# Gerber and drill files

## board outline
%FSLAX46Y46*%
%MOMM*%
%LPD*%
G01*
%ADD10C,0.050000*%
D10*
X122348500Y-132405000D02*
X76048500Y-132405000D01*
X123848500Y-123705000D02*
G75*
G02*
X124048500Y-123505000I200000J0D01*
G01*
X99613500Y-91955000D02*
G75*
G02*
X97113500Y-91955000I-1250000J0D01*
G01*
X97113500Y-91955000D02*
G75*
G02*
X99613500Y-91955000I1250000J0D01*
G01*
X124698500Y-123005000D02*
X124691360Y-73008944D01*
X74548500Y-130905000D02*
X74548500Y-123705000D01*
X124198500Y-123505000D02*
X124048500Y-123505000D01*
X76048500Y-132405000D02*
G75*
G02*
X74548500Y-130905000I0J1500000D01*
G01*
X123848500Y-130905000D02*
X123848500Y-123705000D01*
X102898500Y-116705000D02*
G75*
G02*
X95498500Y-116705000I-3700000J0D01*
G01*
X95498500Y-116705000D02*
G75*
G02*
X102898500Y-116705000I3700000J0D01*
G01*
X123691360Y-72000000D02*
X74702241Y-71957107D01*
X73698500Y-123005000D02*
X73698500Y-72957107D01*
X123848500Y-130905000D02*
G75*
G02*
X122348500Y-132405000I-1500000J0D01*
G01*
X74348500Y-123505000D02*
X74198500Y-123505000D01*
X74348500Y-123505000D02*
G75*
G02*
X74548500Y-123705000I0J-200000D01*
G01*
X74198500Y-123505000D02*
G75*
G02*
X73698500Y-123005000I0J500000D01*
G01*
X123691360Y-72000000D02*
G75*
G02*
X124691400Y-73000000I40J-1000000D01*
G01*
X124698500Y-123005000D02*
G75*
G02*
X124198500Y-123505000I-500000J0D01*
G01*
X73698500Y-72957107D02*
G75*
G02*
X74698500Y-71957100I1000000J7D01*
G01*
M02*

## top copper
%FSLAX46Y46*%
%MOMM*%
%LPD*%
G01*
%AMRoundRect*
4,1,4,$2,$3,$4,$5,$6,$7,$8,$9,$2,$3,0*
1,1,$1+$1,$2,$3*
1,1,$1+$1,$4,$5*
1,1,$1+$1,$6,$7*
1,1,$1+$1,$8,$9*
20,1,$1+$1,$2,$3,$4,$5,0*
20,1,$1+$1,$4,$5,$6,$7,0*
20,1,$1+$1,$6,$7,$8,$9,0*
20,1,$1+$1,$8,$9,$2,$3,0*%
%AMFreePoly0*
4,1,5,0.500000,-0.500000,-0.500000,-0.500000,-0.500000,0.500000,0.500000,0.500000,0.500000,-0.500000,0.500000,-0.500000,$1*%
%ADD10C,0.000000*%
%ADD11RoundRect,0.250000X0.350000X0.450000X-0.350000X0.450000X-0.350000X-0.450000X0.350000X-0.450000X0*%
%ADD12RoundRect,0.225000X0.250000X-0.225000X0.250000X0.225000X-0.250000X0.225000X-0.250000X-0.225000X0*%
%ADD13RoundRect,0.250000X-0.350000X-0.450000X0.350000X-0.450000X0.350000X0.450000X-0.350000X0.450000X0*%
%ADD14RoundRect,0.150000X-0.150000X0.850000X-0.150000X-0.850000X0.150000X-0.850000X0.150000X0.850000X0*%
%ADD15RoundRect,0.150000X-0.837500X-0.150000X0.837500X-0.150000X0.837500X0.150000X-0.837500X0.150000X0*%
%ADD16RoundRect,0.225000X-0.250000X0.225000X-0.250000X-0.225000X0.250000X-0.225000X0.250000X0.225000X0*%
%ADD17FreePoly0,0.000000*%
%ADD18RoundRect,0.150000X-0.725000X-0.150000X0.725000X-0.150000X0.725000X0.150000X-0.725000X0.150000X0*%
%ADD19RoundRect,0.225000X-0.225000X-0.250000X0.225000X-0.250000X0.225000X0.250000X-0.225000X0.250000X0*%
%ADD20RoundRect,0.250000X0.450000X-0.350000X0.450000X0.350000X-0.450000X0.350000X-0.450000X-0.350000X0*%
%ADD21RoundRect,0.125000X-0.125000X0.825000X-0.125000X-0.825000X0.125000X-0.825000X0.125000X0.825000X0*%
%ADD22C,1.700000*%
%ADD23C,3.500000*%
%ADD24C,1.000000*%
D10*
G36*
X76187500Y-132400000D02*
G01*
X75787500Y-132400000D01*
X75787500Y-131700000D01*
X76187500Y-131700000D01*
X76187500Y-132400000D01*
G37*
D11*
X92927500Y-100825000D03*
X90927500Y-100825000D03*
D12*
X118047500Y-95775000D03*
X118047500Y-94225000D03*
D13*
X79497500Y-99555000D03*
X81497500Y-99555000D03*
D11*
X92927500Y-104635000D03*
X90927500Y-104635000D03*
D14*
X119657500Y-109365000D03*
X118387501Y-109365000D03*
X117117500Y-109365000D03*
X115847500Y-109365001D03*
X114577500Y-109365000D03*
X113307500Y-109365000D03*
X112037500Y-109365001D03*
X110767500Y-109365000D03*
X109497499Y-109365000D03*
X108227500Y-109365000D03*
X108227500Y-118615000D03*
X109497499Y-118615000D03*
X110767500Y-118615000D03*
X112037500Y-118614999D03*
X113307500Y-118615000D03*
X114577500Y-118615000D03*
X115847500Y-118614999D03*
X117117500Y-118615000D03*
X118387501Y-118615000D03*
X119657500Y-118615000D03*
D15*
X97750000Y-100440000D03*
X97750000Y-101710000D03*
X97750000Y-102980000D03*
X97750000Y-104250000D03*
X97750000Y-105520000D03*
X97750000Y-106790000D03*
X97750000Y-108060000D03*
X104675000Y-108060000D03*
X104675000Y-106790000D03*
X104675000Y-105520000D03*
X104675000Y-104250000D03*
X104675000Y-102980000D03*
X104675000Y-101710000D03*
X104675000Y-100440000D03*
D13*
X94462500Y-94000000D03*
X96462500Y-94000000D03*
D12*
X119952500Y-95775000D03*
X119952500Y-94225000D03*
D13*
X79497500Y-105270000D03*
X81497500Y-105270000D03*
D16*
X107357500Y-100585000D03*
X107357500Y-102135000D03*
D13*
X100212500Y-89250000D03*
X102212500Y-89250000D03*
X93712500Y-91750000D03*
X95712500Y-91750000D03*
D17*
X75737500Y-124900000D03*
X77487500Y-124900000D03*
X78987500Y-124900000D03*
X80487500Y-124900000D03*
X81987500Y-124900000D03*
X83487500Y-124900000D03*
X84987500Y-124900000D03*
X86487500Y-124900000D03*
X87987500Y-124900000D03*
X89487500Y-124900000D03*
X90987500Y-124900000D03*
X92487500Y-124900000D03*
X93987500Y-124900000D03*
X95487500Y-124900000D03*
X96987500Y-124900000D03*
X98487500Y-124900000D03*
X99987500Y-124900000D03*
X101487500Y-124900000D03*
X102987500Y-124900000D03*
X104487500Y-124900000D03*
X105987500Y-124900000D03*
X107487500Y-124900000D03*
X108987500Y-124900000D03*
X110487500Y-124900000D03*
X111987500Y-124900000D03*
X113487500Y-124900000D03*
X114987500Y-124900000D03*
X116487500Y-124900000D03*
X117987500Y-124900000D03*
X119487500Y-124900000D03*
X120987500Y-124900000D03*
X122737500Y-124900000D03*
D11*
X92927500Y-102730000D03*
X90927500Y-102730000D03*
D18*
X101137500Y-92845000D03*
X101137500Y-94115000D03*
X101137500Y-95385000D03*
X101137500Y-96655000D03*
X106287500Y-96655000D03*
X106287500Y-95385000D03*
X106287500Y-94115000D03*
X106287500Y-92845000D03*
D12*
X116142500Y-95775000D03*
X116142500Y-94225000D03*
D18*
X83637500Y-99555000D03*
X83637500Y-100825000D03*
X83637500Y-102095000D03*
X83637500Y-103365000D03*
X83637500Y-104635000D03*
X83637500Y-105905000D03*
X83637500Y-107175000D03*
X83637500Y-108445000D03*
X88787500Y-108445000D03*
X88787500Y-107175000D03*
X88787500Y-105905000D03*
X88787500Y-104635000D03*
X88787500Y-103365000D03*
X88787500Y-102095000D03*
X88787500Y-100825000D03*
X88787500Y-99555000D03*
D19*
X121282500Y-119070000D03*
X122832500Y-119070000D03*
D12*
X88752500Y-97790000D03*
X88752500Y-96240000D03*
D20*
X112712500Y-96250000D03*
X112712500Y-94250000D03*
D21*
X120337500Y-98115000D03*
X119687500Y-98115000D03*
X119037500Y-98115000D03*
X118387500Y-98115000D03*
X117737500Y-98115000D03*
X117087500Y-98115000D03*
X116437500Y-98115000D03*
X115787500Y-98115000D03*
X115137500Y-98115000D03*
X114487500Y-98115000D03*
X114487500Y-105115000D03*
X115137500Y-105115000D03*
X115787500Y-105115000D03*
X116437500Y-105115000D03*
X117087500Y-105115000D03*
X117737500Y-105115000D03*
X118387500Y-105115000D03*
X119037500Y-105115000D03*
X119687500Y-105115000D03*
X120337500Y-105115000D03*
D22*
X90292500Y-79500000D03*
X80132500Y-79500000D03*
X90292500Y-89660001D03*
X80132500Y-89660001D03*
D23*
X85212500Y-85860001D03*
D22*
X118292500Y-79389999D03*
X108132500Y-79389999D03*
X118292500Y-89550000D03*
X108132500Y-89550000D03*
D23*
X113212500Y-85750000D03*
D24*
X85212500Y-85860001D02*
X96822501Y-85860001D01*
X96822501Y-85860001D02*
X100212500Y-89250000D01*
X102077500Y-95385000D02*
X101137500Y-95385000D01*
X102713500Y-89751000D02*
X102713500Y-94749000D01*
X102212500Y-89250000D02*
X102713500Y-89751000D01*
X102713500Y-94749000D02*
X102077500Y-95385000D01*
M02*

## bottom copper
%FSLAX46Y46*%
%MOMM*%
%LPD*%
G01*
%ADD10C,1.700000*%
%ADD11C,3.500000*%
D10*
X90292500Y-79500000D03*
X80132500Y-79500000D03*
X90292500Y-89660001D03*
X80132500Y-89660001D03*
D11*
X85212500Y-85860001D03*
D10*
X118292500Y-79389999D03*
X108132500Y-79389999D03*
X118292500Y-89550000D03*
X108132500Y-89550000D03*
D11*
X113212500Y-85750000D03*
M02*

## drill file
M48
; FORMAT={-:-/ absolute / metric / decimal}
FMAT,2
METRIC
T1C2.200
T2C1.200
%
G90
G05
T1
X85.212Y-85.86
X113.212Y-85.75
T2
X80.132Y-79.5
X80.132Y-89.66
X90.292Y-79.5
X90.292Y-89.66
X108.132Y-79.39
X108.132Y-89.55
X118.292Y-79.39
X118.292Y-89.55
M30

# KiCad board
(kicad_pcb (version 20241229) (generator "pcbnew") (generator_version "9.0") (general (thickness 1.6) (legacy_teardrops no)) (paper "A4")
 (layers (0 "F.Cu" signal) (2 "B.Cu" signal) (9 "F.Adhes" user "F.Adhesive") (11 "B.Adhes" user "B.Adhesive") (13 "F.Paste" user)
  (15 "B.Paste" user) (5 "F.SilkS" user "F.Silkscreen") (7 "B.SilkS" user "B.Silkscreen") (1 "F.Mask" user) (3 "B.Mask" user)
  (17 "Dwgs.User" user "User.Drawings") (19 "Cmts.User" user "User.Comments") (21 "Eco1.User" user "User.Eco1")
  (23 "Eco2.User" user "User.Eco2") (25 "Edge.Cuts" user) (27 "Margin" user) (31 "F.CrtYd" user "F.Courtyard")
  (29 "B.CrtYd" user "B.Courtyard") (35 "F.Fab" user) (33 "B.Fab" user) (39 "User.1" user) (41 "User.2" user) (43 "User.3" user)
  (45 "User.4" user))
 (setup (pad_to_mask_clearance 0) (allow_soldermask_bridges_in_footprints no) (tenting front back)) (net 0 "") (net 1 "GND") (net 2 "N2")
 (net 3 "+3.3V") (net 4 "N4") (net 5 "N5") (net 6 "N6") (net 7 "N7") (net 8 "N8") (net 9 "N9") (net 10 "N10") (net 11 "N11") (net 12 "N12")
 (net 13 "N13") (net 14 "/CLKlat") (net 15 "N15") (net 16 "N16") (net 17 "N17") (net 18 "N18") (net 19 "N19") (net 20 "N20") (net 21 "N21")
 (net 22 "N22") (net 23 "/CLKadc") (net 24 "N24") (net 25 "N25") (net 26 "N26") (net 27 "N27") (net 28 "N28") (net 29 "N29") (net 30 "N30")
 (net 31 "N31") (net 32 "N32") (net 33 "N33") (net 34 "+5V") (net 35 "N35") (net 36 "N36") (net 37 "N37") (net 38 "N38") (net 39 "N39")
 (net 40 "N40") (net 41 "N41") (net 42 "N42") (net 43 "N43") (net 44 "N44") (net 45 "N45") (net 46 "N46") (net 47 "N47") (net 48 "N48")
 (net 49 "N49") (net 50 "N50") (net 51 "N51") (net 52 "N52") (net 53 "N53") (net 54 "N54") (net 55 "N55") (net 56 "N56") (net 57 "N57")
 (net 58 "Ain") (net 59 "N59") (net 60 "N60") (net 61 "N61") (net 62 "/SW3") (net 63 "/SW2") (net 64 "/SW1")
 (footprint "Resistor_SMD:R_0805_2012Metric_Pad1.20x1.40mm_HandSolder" (layer "F.Cu") (at 91.9275 100.825 180)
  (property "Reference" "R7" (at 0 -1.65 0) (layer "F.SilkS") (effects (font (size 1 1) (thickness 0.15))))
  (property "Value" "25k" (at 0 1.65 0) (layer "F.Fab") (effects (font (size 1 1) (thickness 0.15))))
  (pad "1" smd roundrect (at -1 0 180) (size 1.2 1.4) (layers "F.Cu" "F.Mask" "F.Paste") (roundrect_rratio 0.208333) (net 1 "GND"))
  (pad "2" smd roundrect (at 1 0 180) (size 1.2 1.4) (layers "F.Cu" "F.Mask" "F.Paste") (roundrect_rratio 0.208333) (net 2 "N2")))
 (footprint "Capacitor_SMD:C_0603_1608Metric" (layer "F.Cu") (at 118.0475 95 90)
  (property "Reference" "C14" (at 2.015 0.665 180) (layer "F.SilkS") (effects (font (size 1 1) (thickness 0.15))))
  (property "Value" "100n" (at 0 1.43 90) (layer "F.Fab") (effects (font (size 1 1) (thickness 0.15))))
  (pad "1" smd roundrect (at -0.775 0 90) (size 0.9 0.95) (layers "F.Cu" "F.Mask" "F.Paste") (roundrect_rratio 0.25) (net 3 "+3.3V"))
  (pad "2" smd roundrect (at 0.775 0 90) (size 0.9 0.95) (layers "F.Cu" "F.Mask" "F.Paste") (roundrect_rratio 0.25) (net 1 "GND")))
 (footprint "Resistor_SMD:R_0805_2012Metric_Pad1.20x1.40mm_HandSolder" (layer "F.Cu") (at 80.4975 99.555)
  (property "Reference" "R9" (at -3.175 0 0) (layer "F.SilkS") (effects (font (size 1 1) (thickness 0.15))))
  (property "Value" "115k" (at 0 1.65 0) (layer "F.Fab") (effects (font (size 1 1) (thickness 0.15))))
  (pad "1" smd roundrect (at -1 0) (size 1.2 1.4) (layers "F.Cu" "F.Mask" "F.Paste") (roundrect_rratio 0.208333) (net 1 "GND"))
  (pad "2" smd roundrect (at 1 0) (size 1.2 1.4) (layers "F.Cu" "F.Mask" "F.Paste") (roundrect_rratio 0.208333) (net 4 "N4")))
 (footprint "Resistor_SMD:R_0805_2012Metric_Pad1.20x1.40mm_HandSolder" (layer "F.Cu") (at 91.9275 104.635 180)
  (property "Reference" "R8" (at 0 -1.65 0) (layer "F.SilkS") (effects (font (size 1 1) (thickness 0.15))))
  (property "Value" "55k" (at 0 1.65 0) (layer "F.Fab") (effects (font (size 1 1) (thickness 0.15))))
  (pad "1" smd roundrect (at -1 0 180) (size 1.2 1.4) (layers "F.Cu" "F.Mask" "F.Paste") (roundrect_rratio 0.208333) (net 1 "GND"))
  (pad "2" smd roundrect (at 1 0 180) (size 1.2 1.4) (layers "F.Cu" "F.Mask" "F.Paste") (roundrect_rratio 0.208333) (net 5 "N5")))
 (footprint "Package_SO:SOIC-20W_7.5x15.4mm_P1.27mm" (layer "F.Cu") (at 113.9425 113.99 -90)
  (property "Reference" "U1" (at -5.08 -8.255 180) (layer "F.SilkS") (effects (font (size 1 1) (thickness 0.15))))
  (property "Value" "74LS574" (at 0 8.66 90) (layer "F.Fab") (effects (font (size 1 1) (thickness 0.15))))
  (pad "1" smd roundrect (at -4.625 -5.715 270) (size 2 0.6) (layers "F.Cu" "F.Mask" "F.Paste") (roundrect_rratio 0.25) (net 1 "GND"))
  (pad "2" smd roundrect (at -4.625 -4.445001 270) (size 2 0.6) (layers "F.Cu" "F.Mask" "F.Paste") (roundrect_rratio 0.25) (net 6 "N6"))
  (pad "3" smd roundrect (at -4.625 -3.175 270) (size 2 0.6) (layers "F.Cu" "F.Mask" "F.Paste") (roundrect_rratio 0.25) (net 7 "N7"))
  (pad "4" smd roundrect (at -4.624999 -1.905 270) (size 2 0.6) (layers "F.Cu" "F.Mask" "F.Paste") (roundrect_rratio 0.25) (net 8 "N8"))
  (pad "5" smd roundrect (at -4.625 -0.635 270) (size 2 0.6) (layers "F.Cu" "F.Mask" "F.Paste") (roundrect_rratio 0.25) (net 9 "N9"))
  (pad "6" smd roundrect (at -4.625 0.635 270) (size 2 0.6) (layers "F.Cu" "F.Mask" "F.Paste") (roundrect_rratio 0.25) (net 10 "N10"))
  (pad "7" smd roundrect (at -4.624999 1.905 270) (size 2 0.6) (layers "F.Cu" "F.Mask" "F.Paste") (roundrect_rratio 0.25) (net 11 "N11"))
  (pad "8" smd roundrect (at -4.625 3.175 270) (size 2 0.6) (layers "F.Cu" "F.Mask" "F.Paste") (roundrect_rratio 0.25) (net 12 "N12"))
  (pad "9" smd roundrect (at -4.625 4.445001 270) (size 2 0.6) (layers "F.Cu" "F.Mask" "F.Paste") (roundrect_rratio 0.25) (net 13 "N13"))
  (pad "10" smd roundrect (at -4.625 5.715 270) (size 2 0.6) (layers "F.Cu" "F.Mask" "F.Paste") (roundrect_rratio 0.25) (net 1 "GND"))
  (pad "11" smd roundrect (at 4.625 5.715 270) (size 2 0.6) (layers "F.Cu" "F.Mask" "F.Paste") (roundrect_rratio 0.25) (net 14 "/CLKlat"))
  (pad "12" smd roundrect (at 4.625 4.445001 270) (size 2 0.6) (layers "F.Cu" "F.Mask" "F.Paste") (roundrect_rratio 0.25) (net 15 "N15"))
  (pad "13" smd roundrect (at 4.625 3.175 270) (size 2 0.6) (layers "F.Cu" "F.Mask" "F.Paste") (roundrect_rratio 0.25) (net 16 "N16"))
  (pad "14" smd roundrect (at 4.624999 1.905 270) (size 2 0.6) (layers "F.Cu" "F.Mask" "F.Paste") (roundrect_rratio 0.25) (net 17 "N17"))
  (pad "15" smd roundrect (at 4.625 0.635 270) (size 2 0.6) (layers "F.Cu" "F.Mask" "F.Paste") (roundrect_rratio 0.25) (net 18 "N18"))
  (pad "16" smd roundrect (at 4.625 -0.635 270) (size 2 0.6) (layers "F.Cu" "F.Mask" "F.Paste") (roundrect_rratio 0.25) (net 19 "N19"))
  (pad "17" smd roundrect (at 4.624999 -1.905 270) (size 2 0.6) (layers "F.Cu" "F.Mask" "F.Paste") (roundrect_rratio 0.25) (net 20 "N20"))
  (pad "18" smd roundrect (at 4.625 -3.175 270) (size 2 0.6) (layers "F.Cu" "F.Mask" "F.Paste") (roundrect_rratio 0.25) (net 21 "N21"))
  (pad "19" smd roundrect (at 4.625 -4.445001 270) (size 2 0.6) (layers "F.Cu" "F.Mask" "F.Paste") (roundrect_rratio 0.25) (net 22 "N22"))
  (pad "20" smd roundrect (at 4.625 -5.715 270) (size 2 0.6) (layers "F.Cu" "F.Mask" "F.Paste") (roundrect_rratio 0.25) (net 3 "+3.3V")))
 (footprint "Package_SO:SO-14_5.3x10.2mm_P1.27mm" (layer "F.Cu") (at 101.2125 104.25)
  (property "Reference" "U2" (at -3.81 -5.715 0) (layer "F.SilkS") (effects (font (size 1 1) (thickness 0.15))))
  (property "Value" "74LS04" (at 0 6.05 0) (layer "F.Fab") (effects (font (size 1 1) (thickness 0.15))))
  (pad "1" smd roundrect (at -3.4625 -3.81) (size 1.975 0.6) (layers "F.Cu" "F.Mask" "F.Paste") (roundrect_rratio 0.25) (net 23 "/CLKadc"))
  (pad "2" smd roundrect (at -3.4625 -2.54) (size 1.975 0.6) (layers "F.Cu" "F.Mask" "F.Paste") (roundrect_rratio 0.25) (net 14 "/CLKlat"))
  (pad "3" smd roundrect (at -3.4625 -1.27) (size 1.975 0.6) (layers "F.Cu" "F.Mask" "F.Paste") (roundrect_rratio 0.25) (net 1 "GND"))
  (pad "4" smd roundrect (at -3.4625 0) (size 1.975 0.6) (layers "F.Cu" "F.Mask" "F.Paste") (roundrect_rratio 0.25) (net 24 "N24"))
  (pad "5" smd roundrect (at -3.4625 1.27) (size 1.975 0.6) (layers "F.Cu" "F.Mask" "F.Paste") (roundrect_rratio 0.25) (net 1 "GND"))
  (pad "6" smd roundrect (at -3.4625 2.54) (size 1.975 0.6) (layers "F.Cu" "F.Mask" "F.Paste") (roundrect_rratio 0.25) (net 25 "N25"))
  (pad "7" smd roundrect (at -3.4625 3.81) (size 1.975 0.6) (layers "F.Cu" "F.Mask" "F.Paste") (roundrect_rratio 0.25) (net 1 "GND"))
  (pad "8" smd roundrect (at 3.4625 3.81) (size 1.975 0.6) (layers "F.Cu" "F.Mask" "F.Paste") (roundrect_rratio 0.25) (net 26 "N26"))
  (pad "9" smd roundrect (at 3.4625 2.54) (size 1.975 0.6) (layers "F.Cu" "F.Mask" "F.Paste") (roundrect_rratio 0.25) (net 1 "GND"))
  (pad "10" smd roundrect (at 3.4625 1.27) (size 1.975 0.6) (layers "F.Cu" "F.Mask" "F.Paste") (roundrect_rratio 0.25) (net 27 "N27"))
  (pad "11" smd roundrect (at 3.4625 0) (size 1.975 0.6) (layers "F.Cu" "F.Mask" "F.Paste") (roundrect_rratio 0.25) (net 1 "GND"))
  (pad "12" smd roundrect (at 3.4625 -1.27) (size 1.975 0.6) (layers "F.Cu" "F.Mask" "F.Paste") (roundrect_rratio 0.25) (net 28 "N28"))
  (pad "13" smd roundrect (at 3.4625 -2.54) (size 1.975 0.6) (layers "F.Cu" "F.Mask" "F.Paste") (roundrect_rratio 0.25) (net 1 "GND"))
  (pad "14" smd roundrect (at 3.4625 -3.81) (size 1.975 0.6) (layers "F.Cu" "F.Mask" "F.Paste") (roundrect_rratio 0.25) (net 3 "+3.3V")))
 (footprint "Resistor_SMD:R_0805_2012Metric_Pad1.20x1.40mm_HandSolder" (layer "F.Cu") (at 95.4625 94)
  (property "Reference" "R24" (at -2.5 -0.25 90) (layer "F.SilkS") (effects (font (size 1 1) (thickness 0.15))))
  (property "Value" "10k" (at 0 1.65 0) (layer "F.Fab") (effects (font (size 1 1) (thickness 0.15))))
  (pad "1" smd roundrect (at -1 0) (size 1.2 1.4) (layers "F.Cu" "F.Mask" "F.Paste") (roundrect_rratio 0.208333) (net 3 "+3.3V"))
  (pad "2" smd roundrect (at 1 0) (size 1.2 1.4) (layers "F.Cu" "F.Mask" "F.Paste") (roundrect_rratio 0.208333) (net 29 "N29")))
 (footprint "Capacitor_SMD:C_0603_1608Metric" (layer "F.Cu") (at 119.9525 95 90)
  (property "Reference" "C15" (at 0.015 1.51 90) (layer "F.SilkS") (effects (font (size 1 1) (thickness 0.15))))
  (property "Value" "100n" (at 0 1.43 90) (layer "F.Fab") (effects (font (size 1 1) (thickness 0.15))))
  (pad "1" smd roundrect (at -0.775 0 90) (size 0.9 0.95) (layers "F.Cu" "F.Mask" "F.Paste") (roundrect_rratio 0.25) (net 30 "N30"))
  (pad "2" smd roundrect (at 0.775 0 90) (size 0.9 0.95) (layers "F.Cu" "F.Mask" "F.Paste") (roundrect_rratio 0.25) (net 1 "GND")))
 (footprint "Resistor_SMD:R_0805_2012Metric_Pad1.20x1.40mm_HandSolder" (layer "F.Cu") (at 80.4975 105.27)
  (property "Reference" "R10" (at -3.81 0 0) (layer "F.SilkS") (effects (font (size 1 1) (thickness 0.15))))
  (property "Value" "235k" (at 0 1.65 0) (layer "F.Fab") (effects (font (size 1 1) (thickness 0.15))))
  (pad "1" smd roundrect (at -1 0) (size 1.2 1.4) (layers "F.Cu" "F.Mask" "F.Paste") (roundrect_rratio 0.208333) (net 1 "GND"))
  (pad "2" smd roundrect (at 1 0) (size 1.2 1.4) (layers "F.Cu" "F.Mask" "F.Paste") (roundrect_rratio 0.208333) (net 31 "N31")))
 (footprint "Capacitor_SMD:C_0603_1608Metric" (layer "F.Cu") (at 107.3575 101.36 -90)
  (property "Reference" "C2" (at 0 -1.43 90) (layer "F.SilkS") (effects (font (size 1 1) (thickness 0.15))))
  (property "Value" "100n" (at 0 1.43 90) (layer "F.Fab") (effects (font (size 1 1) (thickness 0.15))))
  (pad "1" smd roundrect (at -0.775 0 270) (size 0.9 0.95) (layers "F.Cu" "F.Mask" "F.Paste") (roundrect_rratio 0.25) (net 3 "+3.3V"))
  (pad "2" smd roundrect (at 0.775 0 270) (size 0.9 0.95) (layers "F.Cu" "F.Mask" "F.Paste") (roundrect_rratio 0.25) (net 1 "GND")))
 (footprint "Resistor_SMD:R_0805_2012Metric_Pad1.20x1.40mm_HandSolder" (layer "F.Cu") (at 101.2125 89.25)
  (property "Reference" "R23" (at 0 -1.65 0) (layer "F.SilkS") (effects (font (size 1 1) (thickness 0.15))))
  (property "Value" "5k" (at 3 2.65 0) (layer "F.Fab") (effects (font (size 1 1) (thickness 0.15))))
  (pad "1" smd roundrect (at -1 0) (size 1.2 1.4) (layers "F.Cu" "F.Mask" "F.Paste") (roundrect_rratio 0.208333) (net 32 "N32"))
  (pad "2" smd roundrect (at 1 0) (size 1.2 1.4) (layers "F.Cu" "F.Mask" "F.Paste") (roundrect_rratio 0.208333) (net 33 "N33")))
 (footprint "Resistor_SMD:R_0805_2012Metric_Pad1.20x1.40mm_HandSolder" (layer "F.Cu") (at 94.7125 91.75)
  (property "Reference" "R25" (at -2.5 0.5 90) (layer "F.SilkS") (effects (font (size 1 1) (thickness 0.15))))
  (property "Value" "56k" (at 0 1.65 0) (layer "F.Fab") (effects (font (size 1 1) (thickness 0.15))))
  (pad "1" smd roundrect (at -1 0) (size 1.2 1.4) (layers "F.Cu" "F.Mask" "F.Paste") (roundrect_rratio 0.208333) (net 29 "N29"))
  (pad "2" smd roundrect (at 1 0) (size 1.2 1.4) (layers "F.Cu" "F.Mask" "F.Paste") (roundrect_rratio 0.208333) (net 1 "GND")))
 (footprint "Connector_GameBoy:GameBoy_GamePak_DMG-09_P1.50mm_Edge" (layer "F.Cu") (at 99.2375 132.4)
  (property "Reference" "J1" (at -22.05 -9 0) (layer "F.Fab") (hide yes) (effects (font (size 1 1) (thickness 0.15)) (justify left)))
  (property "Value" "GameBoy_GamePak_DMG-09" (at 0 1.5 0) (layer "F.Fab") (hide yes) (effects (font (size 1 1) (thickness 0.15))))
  (fp_poly (pts (xy -23.05 0) (xy -23.45 0) (xy -23.45 -0.7) (xy -23.05 -0.7)) (stroke (width 0) (type solid)) (fill yes) (layer "F.Cu"))
  (pad "1" smd custom (at -23.5 -7.5) (size 1 1) (layers "F.Cu") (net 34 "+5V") (zone_connect 0) (options (clearance outline) (anchor rect))
   (primitives))
  (pad "2" smd custom (at -21.75 -7.5) (size 1 1) (layers "F.Cu") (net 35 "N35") (options (clearance outline) (anchor rect)) (primitives))
  (pad "3" smd custom (at -20.25 -7.5) (size 1 1) (layers "F.Cu") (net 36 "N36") (options (clearance outline) (anchor rect)) (primitives))
  (pad "4" smd custom (at -18.75 -7.5) (size 1 1) (layers "F.Cu") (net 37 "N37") (options (clearance outline) (anchor rect)) (primitives))
  (pad "5" smd custom (at -17.25 -7.5) (size 1 1) (layers "F.Cu") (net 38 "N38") (options (clearance outline) (anchor rect)) (primitives))
  (pad "6" smd custom (at -15.75 -7.5) (size 1 1) (layers "F.Cu") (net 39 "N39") (options (clearance outline) (anchor rect)) (primitives))
  (pad "7" smd custom (at -14.25 -7.5) (size 1 1) (layers "F.Cu") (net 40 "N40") (options (clearance outline) (anchor rect)) (primitives))
  (pad "8" smd custom (at -12.75 -7.5) (size 1 1) (layers "F.Cu") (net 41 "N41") (options (clearance outline) (anchor rect)) (primitives))
  (pad "9" smd custom (at -11.25 -7.5) (size 1 1) (layers "F.Cu") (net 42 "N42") (options (clearance outline) (anchor rect)) (primitives))
  (pad "10" smd custom (at -9.75 -7.5) (size 1 1) (layers "F.Cu") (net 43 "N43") (options (clearance outline) (anchor rect)) (primitives))
  (pad "11" smd custom (at -8.25 -7.5) (size 1 1) (layers "F.Cu") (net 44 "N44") (options (clearance outline) (anchor rect)) (primitives))
  (pad "12" smd custom (at -6.75 -7.5) (size 1 1) (layers "F.Cu") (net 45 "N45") (options (clearance outline) (anchor rect)) (primitives))
  (pad "13" smd custom (at -5.25 -7.5) (size 1 1) (layers "F.Cu") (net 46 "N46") (options (clearance outline) (anchor rect)) (primitives))
  (pad "14" smd custom (at -3.75 -7.5) (size 1 1) (layers "F.Cu") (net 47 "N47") (options (clearance outline) (anchor rect)) (primitives))
  (pad "15" smd custom (at -2.25 -7.5) (size 1 1) (layers "F.Cu") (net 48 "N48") (options (clearance outline) (anchor rect)) (primitives))
  (pad "16" smd custom (at -0.75 -7.5) (size 1 1) (layers "F.Cu") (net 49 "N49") (options (clearance outline) (anchor rect)) (primitives))
  (pad "17" smd custom (at 0.75 -7.5) (size 1 1) (layers "F.Cu") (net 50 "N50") (options (clearance outline) (anchor rect)) (primitives))
  (pad "18" smd custom (at 2.25 -7.5) (size 1 1) (layers "F.Cu") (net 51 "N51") (options (clearance outline) (anchor rect)) (primitives))
  (pad "19" smd custom (at 3.75 -7.5) (size 1 1) (layers "F.Cu") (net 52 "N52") (options (clearance outline) (anchor rect)) (primitives))
  (pad "20" smd custom (at 5.25 -7.5) (size 1 1) (layers "F.Cu") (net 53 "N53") (options (clearance outline) (anchor rect)) (primitives))
  (pad "21" smd custom (at 6.75 -7.5) (size 1 1) (layers "F.Cu") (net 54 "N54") (options (clearance outline) (anchor rect)) (primitives))
  (pad "22" smd custom (at 8.25 -7.5) (size 1 1) (layers "F.Cu") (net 22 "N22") (options (clearance outline) (anchor rect)) (primitives))
  (pad "23" smd custom (at 9.75 -7.5) (size 1 1) (layers "F.Cu") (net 21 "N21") (options (clearance outline) (anchor rect)) (primitives))
  (pad "24" smd custom (at 11.25 -7.5) (size 1 1) (layers "F.Cu") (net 20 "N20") (options (clearance outline) (anchor rect)) (primitives))
  (pad "25" smd custom (at 12.75 -7.5) (size 1 1) (layers "F.Cu") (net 19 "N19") (options (clearance outline) (anchor rect)) (primitives))
  (pad "26" smd custom (at 14.25 -7.5) (size 1 1) (layers "F.Cu") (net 18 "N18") (options (clearance outline) (anchor rect)) (primitives))
  (pad "27" smd custom (at 15.75 -7.5) (size 1 1) (layers "F.Cu") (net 17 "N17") (options (clearance outline) (anchor rect)) (primitives))
  (pad "28" smd custom (at 17.25 -7.5) (size 1 1) (layers "F.Cu") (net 16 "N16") (options (clearance outline) (anchor rect)) (primitives))
  (pad "29" smd custom (at 18.75 -7.5) (size 1 1) (layers "F.Cu") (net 15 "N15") (options (clearance outline) (anchor rect)) (primitives))
  (pad "30" smd custom (at 20.25 -7.5) (size 1 1) (layers "F.Cu") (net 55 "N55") (options (clearance outline) (anchor rect)) (primitives))
  (pad "31" smd custom (at 21.75 -7.5) (size 1 1) (layers "F.Cu") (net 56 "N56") (options (clearance outline) (anchor rect)) (primitives))
  (pad "32" smd custom (at 23.5 -7.5) (size 1 1) (layers "F.Cu") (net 1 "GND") (zone_connect 0) (options (clearance outline) (anchor rect))
   (primitives)))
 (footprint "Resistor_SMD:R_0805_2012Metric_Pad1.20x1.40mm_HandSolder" (layer "F.Cu") (at 91.9275 102.73 180)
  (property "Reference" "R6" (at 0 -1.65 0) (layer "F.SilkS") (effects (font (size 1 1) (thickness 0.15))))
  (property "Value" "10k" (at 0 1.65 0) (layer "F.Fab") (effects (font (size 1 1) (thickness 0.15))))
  (pad "1" smd roundrect (at -1 0 180) (size 1.2 1.4) (layers "F.Cu" "F.Mask" "F.Paste") (roundrect_rratio 0.208333) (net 1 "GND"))
  (pad "2" smd roundrect (at 1 0 180) (size 1.2 1.4) (layers "F.Cu" "F.Mask" "F.Paste") (roundrect_rratio 0.208333) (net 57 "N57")))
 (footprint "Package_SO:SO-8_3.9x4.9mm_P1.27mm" (layer "F.Cu") (at 103.7125 94.75)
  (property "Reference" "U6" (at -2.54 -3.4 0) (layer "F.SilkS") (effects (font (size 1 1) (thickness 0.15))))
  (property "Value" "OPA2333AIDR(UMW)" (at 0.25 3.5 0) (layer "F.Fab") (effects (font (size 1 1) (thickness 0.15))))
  (pad "1" smd roundrect (at -2.575 -1.905) (size 1.75 0.6) (layers "F.Cu" "F.Mask" "F.Paste") (roundrect_rratio 0.25) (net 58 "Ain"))
  (pad "2" smd roundrect (at -2.575 -0.635) (size 1.75 0.6) (layers "F.Cu" "F.Mask" "F.Paste") (roundrect_rratio 0.25) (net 29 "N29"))
  (pad "3" smd roundrect (at -2.575 0.635) (size 1.75 0.6) (layers "F.Cu" "F.Mask" "F.Paste") (roundrect_rratio 0.25) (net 33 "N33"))
  (pad "4" smd roundrect (at -2.575 1.905) (size 1.75 0.6) (layers "F.Cu" "F.Mask" "F.Paste") (roundrect_rratio 0.25))
  (pad "5" smd roundrect (at 2.575 1.905) (size 1.75 0.6) (layers "F.Cu" "F.Mask" "F.Paste") (roundrect_rratio 0.25))
  (pad "6" smd roundrect (at 2.575 0.635) (size 1.75 0.6) (layers "F.Cu" "F.Mask" "F.Paste") (roundrect_rratio 0.25))
  (pad "7" smd roundrect (at 2.575 -0.635) (size 1.75 0.6) (layers "F.Cu" "F.Mask" "F.Paste") (roundrect_rratio 0.25))
  (pad "8" smd roundrect (at 2.575 -1.905) (size 1.75 0.6) (layers "F.Cu" "F.Mask" "F.Paste") (roundrect_rratio 0.25)))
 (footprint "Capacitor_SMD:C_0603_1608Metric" (layer "F.Cu") (at 116.1425 95 90)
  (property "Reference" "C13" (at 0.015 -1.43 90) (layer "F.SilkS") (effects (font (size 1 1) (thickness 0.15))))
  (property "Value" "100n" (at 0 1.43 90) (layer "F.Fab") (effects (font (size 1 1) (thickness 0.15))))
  (pad "1" smd roundrect (at -0.775 0 90) (size 0.9 0.95) (layers "F.Cu" "F.Mask" "F.Paste") (roundrect_rratio 0.25) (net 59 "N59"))
  (pad "2" smd roundrect (at 0.775 0 90) (size 0.9 0.95) (layers "F.Cu" "F.Mask" "F.Paste") (roundrect_rratio 0.25) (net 1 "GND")))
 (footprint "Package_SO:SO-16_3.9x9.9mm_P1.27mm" (layer "F.Cu") (at 86.2125 104)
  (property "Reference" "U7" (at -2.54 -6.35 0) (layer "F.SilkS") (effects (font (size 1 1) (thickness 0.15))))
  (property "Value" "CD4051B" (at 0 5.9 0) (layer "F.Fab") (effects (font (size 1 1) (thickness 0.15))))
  (pad "1" smd roundrect (at -2.575 -4.445) (size 1.75 0.6) (layers "F.Cu" "F.Mask" "F.Paste") (roundrect_rratio 0.25) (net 4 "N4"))
  (pad "2" smd roundrect (at -2.575 -3.175) (size 1.75 0.6) (layers "F.Cu" "F.Mask" "F.Paste") (roundrect_rratio 0.25) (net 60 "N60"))
  (pad "3" smd roundrect (at -2.575 -1.905) (size 1.75 0.6) (layers "F.Cu" "F.Mask" "F.Paste") (roundrect_rratio 0.25) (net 33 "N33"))
  (pad "4" smd roundrect (at -2.575 -0.635) (size 1.75 0.6) (layers "F.Cu" "F.Mask" "F.Paste") (roundrect_rratio 0.25) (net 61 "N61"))
  (pad "5" smd roundrect (at -2.575 0.635) (size 1.75 0.6) (layers "F.Cu" "F.Mask" "F.Paste") (roundrect_rratio 0.25) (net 31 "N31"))
  (pad "6" smd roundrect (at -2.575 1.905) (size 1.75 0.6) (layers "F.Cu" "F.Mask" "F.Paste") (roundrect_rratio 0.25) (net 1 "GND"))
  (pad "7" smd roundrect (at -2.575 3.175) (size 1.75 0.6) (layers "F.Cu" "F.Mask" "F.Paste") (roundrect_rratio 0.25) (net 1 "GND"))
  (pad "8" smd roundrect (at -2.575 4.445) (size 1.75 0.6) (layers "F.Cu" "F.Mask" "F.Paste") (roundrect_rratio 0.25) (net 1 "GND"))
  (pad "9" smd roundrect (at 2.575 4.445) (size 1.75 0.6) (layers "F.Cu" "F.Mask" "F.Paste") (roundrect_rratio 0.25) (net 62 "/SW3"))
  (pad "10" smd roundrect (at 2.575 3.175) (size 1.75 0.6) (layers "F.Cu" "F.Mask" "F.Paste") (roundrect_rratio 0.25) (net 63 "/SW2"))
  (pad "11" smd roundrect (at 2.575 1.905) (size 1.75 0.6) (layers "F.Cu" "F.Mask" "F.Paste") (roundrect_rratio 0.25) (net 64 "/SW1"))
  (pad "12" smd roundrect (at 2.575 0.635) (size 1.75 0.6) (layers "F.Cu" "F.Mask" "F.Paste") (roundrect_rratio 0.25) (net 5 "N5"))
  (pad "13" smd roundrect (at 2.575 -0.635) (size 1.75 0.6) (layers "F.Cu" "F.Mask" "F.Paste") (roundrect_rratio 0.25) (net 1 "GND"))
  (pad "14" smd roundrect (at 2.575 -1.905) (size 1.75 0.6) (layers "F.Cu" "F.Mask" "F.Paste") (roundrect_rratio 0.25) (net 57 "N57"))
  (pad "15" smd roundrect (at 2.575 -3.175) (size 1.75 0.6) (layers "F.Cu" "F.Mask" "F.Paste") (roundrect_rratio 0.25) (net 2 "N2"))
  (pad "16" smd roundrect (at 2.575 -4.445) (size 1.75 0.6) (layers "F.Cu" "F.Mask" "F.Paste") (roundrect_rratio 0.25) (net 3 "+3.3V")))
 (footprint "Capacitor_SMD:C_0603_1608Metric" (layer "F.Cu") (at 122.0575 119.07)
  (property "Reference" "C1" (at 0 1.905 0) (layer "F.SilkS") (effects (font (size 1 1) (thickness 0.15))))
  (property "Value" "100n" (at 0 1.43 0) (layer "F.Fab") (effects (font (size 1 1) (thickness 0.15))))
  (pad "1" smd roundrect (at -0.775 0) (size 0.9 0.95) (layers "F.Cu" "F.Mask" "F.Paste") (roundrect_rratio 0.25) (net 3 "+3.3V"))
  (pad "2" smd roundrect (at 0.775 0) (size 0.9 0.95) (layers "F.Cu" "F.Mask" "F.Paste") (roundrect_rratio 0.25) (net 1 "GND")))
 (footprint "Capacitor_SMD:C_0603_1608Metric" (layer "F.Cu") (at 88.7525 97.015 90)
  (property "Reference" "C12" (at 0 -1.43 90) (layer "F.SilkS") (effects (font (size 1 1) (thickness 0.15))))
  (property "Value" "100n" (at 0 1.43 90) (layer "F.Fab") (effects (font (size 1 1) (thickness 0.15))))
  (pad "1" smd roundrect (at -0.775 0 90) (size 0.9 0.95) (layers "F.Cu" "F.Mask" "F.Paste") (roundrect_rratio 0.25) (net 3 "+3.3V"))
  (pad "2" smd roundrect (at 0.775 0 90) (size 0.9 0.95) (layers "F.Cu" "F.Mask" "F.Paste") (roundrect_rratio 0.25) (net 1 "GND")))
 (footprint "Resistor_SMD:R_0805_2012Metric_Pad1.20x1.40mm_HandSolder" (layer "F.Cu") (at 112.7125 95.25 90)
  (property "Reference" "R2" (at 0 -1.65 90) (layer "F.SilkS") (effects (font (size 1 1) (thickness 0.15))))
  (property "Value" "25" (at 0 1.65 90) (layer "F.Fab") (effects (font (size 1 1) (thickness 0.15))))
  (pad "1" smd roundrect (at -1 0 90) (size 1.2 1.4) (layers "F.Cu" "F.Mask" "F.Paste") (roundrect_rratio 0.208333) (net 59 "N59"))
  (pad "2" smd roundrect (at 1 0 90) (size 1.2 1.4) (layers "F.Cu" "F.Mask" "F.Paste") (roundrect_rratio 0.208333) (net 1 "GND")))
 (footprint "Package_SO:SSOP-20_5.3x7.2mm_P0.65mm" (layer "F.Cu") (at 117.4125 101.615 -90)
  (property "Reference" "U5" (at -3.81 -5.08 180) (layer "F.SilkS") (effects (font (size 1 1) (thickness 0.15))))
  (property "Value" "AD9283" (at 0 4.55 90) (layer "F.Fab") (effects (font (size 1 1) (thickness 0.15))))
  (pad "1" smd roundrect (at -3.5 -2.925 270) (size 1.9 0.5) (layers "F.Cu" "F.Mask" "F.Paste") (roundrect_rratio 0.25) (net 1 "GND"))
  (pad "2" smd roundrect (at -3.5 -2.275 270) (size 1.9 0.5) (layers "F.Cu" "F.Mask" "F.Paste") (roundrect_rratio 0.25) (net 30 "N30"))
  (pad "3" smd roundrect (at -3.5 -1.625 270) (size 1.9 0.5) (layers "F.Cu" "F.Mask" "F.Paste") (roundrect_rratio 0.25) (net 30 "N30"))
  (pad "4" smd roundrect (at -3.5 -0.975 270) (size 1.9 0.5) (layers "F.Cu" "F.Mask" "F.Paste") (roundrect_rratio 0.25) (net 1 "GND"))
  (pad "5" smd roundrect (at -3.5 -0.325 270) (size 1.9 0.5) (layers "F.Cu" "F.Mask" "F.Paste") (roundrect_rratio 0.25) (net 3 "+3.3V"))
  (pad "6" smd roundrect (at -3.5 0.325 270) (size 1.9 0.5) (layers "F.Cu" "F.Mask" "F.Paste") (roundrect_rratio 0.25) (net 59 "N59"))
  (pad "7" smd roundrect (at -3.5 0.975 270) (size 1.9 0.5) (layers "F.Cu" "F.Mask" "F.Paste") (roundrect_rratio 0.25) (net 58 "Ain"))
  (pad "8" smd roundrect (at -3.5 1.625 270) (size 1.9 0.5) (layers "F.Cu" "F.Mask" "F.Paste") (roundrect_rratio 0.25) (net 3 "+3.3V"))
  (pad "9" smd roundrect (at -3.5 2.275 270) (size 1.9 0.5) (layers "F.Cu" "F.Mask" "F.Paste") (roundrect_rratio 0.25) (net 1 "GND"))
  (pad "10" smd roundrect (at -3.5 2.925 270) (size 1.9 0.5) (layers "F.Cu" "F.Mask" "F.Paste") (roundrect_rratio 0.25) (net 23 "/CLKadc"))
  (pad "11" smd roundrect (at 3.5 2.925 270) (size 1.9 0.5) (layers "F.Cu" "F.Mask" "F.Paste") (roundrect_rratio 0.25) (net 13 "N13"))
  (pad "12" smd roundrect (at 3.5 2.275 270) (size 1.9 0.5) (layers "F.Cu" "F.Mask" "F.Paste") (roundrect_rratio 0.25) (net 12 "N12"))
  (pad "13" smd roundrect (at 3.5 1.625 270) (size 1.9 0.5) (layers "F.Cu" "F.Mask" "F.Paste") (roundrect_rratio 0.25) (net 11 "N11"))
  (pad "14" smd roundrect (at 3.5 0.975 270) (size 1.9 0.5) (layers "F.Cu" "F.Mask" "F.Paste") (roundrect_rratio 0.25) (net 10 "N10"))
  (pad "15" smd roundrect (at 3.5 0.325 270) (size 1.9 0.5) (layers "F.Cu" "F.Mask" "F.Paste") (roundrect_rratio 0.25) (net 3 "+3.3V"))
  (pad "16" smd roundrect (at 3.5 -0.325 270) (size 1.9 0.5) (layers "F.Cu" "F.Mask" "F.Paste") (roundrect_rratio 0.25) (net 1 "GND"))
  (pad "17" smd roundrect (at 3.5 -0.975 270) (size 1.9 0.5) (layers "F.Cu" "F.Mask" "F.Paste") (roundrect_rratio 0.25) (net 9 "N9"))
  (pad "18" smd roundrect (at 3.5 -1.625 270) (size 1.9 0.5) (layers "F.Cu" "F.Mask" "F.Paste") (roundrect_rratio 0.25) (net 8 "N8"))
  (pad "19" smd roundrect (at 3.5 -2.275 270) (size 1.9 0.5) (layers "F.Cu" "F.Mask" "F.Paste") (roundrect_rratio 0.25) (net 7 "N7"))
  (pad "20" smd roundrect (at 3.5 -2.925 270) (size 1.9 0.5) (layers "F.Cu" "F.Mask" "F.Paste") (roundrect_rratio 0.25) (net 6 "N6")))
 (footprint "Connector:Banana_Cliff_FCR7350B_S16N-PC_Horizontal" (layer "B.Cu") (at 85.2125 85.860001 -90)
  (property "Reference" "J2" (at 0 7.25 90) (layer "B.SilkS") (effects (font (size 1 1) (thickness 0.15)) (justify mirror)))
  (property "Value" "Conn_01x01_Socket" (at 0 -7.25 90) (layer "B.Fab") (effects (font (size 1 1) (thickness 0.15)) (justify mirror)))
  (pad "" np_thru_hole circle (at -6.360001 -5.08 270) (size 1.7 1.7) (drill 1.2) (layers "*.Cu" "*.Mask"))
  (pad "" np_thru_hole circle (at -6.360001 5.08 270) (size 1.7 1.7) (drill 1.2) (layers "*.Cu" "*.Mask"))
  (pad "" np_thru_hole circle (at 3.8 -5.08 270) (size 1.7 1.7) (drill 1.2) (layers "*.Cu" "*.Mask"))
  (pad "" np_thru_hole circle (at 3.8 5.08 270) (size 1.7 1.7) (drill 1.2) (layers "*.Cu" "*.Mask"))
  (pad "1" thru_hole circle (at 0 0 270) (size 3.5 3.5) (drill 2.2) (layers "*.Cu" "*.Mask") (remove_unused_layers no) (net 32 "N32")))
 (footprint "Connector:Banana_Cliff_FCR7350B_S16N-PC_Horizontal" (layer "B.Cu") (at 113.2125 85.75 -90)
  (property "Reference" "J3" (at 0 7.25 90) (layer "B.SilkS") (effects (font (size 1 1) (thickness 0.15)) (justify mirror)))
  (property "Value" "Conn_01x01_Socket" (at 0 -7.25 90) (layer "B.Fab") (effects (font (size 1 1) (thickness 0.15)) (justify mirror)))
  (pad "" np_thru_hole circle (at -6.360001 -5.08 270) (size 1.7 1.7) (drill 1.2) (layers "*.Cu" "*.Mask"))
  (pad "" np_thru_hole circle (at -6.360001 5.08 270) (size 1.7 1.7) (drill 1.2) (layers "*.Cu" "*.Mask"))
  (pad "" np_thru_hole circle (at 3.8 -5.08 270) (size 1.7 1.7) (drill 1.2) (layers "*.Cu" "*.Mask"))
  (pad "" np_thru_hole circle (at 3.8 5.08 270) (size 1.7 1.7) (drill 1.2) (layers "*.Cu" "*.Mask"))
  (pad "1" thru_hole circle (at 0 0 270) (size 3.5 3.5) (drill 2.2) (layers "*.Cu" "*.Mask") (remove_unused_layers no) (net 1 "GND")))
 (gr_line (start 122.3485 132.405) (end 76.0485 132.405) (stroke (width 0.05) (type solid)) (layer "Edge.Cuts"))
 (gr_arc (start 123.8485 123.705) (mid 123.907079 123.563579) (end 124.0485 123.505) (stroke (width 0.05) (type solid)) (layer "Edge.Cuts"))
 (gr_circle (center 98.3635 91.955) (end 99.6135 91.955) (stroke (width 0.05) (type solid)) (fill no) (layer "Edge.Cuts"))
 (gr_line (start 124.6985 123.005) (end 124.69136 73.008944) (stroke (width 0.05) (type solid)) (layer "Edge.Cuts"))
 (gr_line (start 74.5485 130.905) (end 74.5485 123.705) (stroke (width 0.05) (type solid)) (layer "Edge.Cuts"))
 (gr_line (start 124.1985 123.505) (end 124.0485 123.505) (stroke (width 0.05) (type solid)) (layer "Edge.Cuts"))
 (gr_arc (start 76.0485 132.405) (mid 74.98784 131.96566) (end 74.5485 130.905) (stroke (width 0.05) (type solid)) (layer "Edge.Cuts"))
 (gr_line (start 123.8485 130.905) (end 123.8485 123.705) (stroke (width 0.05) (type solid)) (layer "Edge.Cuts"))
 (gr_circle (center 99.1985 116.705) (end 102.8985 116.705) (stroke (width 0.05) (type solid)) (fill no) (layer "Edge.Cuts"))
 (gr_line (start 123.69136 72) (end 74.702241 71.957107) (stroke (width 0.05) (type solid)) (layer "Edge.Cuts"))
 (gr_line (start 73.6985 123.005) (end 73.6985 72.957107) (stroke (width 0.05) (type solid)) (layer "Edge.Cuts"))
 (gr_arc (start 123.8485 130.905) (mid 123.40916 131.96566) (end 122.3485 132.405) (stroke (width 0.05) (type solid)) (layer "Edge.Cuts"))
 (gr_line (start 74.3485 123.505) (end 74.1985 123.505) (stroke (width 0.05) (type solid)) (layer "Edge.Cuts"))
 (gr_arc (start 74.3485 123.505) (mid 74.489921 123.563579) (end 74.5485 123.705) (stroke (width 0.05) (type solid)) (layer "Edge.Cuts"))
 (gr_arc (start 74.1985 123.505) (mid 73.844947 123.358553) (end 73.6985 123.005) (stroke (width 0.05) (type solid)) (layer "Edge.Cuts"))
 (gr_arc (start 123.69136 72) (mid 124.398467 72.292893) (end 124.69136 73) (stroke (width 0.05) (type solid)) (layer "Edge.Cuts"))
 (gr_arc (start 124.6985 123.005) (mid 124.552053 123.358553) (end 124.1985 123.505) (stroke (width 0.05) (type solid)) (layer "Edge.Cuts"))
 (gr_arc (start 73.6985 72.957107) (mid 73.991393 72.25) (end 74.6985 71.957107) (stroke (width 0.05) (type solid)) (layer "Edge.Cuts"))
 (segment (start 85.2125 85.860001) (end 96.822501 85.860001) (width 1) (layer "F.Cu") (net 32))
 (segment (start 96.822501 85.860001) (end 100.2125 89.25) (width 1) (layer "F.Cu") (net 32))
 (segment (start 102.0775 95.385) (end 101.1375 95.385) (width 1) (layer "F.Cu") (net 33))
 (segment (start 102.7135 89.751) (end 102.7135 94.749) (width 1) (layer "F.Cu") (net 33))
 (segment (start 102.2125 89.25) (end 102.7135 89.751) (width 1) (layer "F.Cu") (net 33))
 (segment (start 102.7135 94.749) (end 102.0775 95.385) (width 1) (layer "F.Cu") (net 33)))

